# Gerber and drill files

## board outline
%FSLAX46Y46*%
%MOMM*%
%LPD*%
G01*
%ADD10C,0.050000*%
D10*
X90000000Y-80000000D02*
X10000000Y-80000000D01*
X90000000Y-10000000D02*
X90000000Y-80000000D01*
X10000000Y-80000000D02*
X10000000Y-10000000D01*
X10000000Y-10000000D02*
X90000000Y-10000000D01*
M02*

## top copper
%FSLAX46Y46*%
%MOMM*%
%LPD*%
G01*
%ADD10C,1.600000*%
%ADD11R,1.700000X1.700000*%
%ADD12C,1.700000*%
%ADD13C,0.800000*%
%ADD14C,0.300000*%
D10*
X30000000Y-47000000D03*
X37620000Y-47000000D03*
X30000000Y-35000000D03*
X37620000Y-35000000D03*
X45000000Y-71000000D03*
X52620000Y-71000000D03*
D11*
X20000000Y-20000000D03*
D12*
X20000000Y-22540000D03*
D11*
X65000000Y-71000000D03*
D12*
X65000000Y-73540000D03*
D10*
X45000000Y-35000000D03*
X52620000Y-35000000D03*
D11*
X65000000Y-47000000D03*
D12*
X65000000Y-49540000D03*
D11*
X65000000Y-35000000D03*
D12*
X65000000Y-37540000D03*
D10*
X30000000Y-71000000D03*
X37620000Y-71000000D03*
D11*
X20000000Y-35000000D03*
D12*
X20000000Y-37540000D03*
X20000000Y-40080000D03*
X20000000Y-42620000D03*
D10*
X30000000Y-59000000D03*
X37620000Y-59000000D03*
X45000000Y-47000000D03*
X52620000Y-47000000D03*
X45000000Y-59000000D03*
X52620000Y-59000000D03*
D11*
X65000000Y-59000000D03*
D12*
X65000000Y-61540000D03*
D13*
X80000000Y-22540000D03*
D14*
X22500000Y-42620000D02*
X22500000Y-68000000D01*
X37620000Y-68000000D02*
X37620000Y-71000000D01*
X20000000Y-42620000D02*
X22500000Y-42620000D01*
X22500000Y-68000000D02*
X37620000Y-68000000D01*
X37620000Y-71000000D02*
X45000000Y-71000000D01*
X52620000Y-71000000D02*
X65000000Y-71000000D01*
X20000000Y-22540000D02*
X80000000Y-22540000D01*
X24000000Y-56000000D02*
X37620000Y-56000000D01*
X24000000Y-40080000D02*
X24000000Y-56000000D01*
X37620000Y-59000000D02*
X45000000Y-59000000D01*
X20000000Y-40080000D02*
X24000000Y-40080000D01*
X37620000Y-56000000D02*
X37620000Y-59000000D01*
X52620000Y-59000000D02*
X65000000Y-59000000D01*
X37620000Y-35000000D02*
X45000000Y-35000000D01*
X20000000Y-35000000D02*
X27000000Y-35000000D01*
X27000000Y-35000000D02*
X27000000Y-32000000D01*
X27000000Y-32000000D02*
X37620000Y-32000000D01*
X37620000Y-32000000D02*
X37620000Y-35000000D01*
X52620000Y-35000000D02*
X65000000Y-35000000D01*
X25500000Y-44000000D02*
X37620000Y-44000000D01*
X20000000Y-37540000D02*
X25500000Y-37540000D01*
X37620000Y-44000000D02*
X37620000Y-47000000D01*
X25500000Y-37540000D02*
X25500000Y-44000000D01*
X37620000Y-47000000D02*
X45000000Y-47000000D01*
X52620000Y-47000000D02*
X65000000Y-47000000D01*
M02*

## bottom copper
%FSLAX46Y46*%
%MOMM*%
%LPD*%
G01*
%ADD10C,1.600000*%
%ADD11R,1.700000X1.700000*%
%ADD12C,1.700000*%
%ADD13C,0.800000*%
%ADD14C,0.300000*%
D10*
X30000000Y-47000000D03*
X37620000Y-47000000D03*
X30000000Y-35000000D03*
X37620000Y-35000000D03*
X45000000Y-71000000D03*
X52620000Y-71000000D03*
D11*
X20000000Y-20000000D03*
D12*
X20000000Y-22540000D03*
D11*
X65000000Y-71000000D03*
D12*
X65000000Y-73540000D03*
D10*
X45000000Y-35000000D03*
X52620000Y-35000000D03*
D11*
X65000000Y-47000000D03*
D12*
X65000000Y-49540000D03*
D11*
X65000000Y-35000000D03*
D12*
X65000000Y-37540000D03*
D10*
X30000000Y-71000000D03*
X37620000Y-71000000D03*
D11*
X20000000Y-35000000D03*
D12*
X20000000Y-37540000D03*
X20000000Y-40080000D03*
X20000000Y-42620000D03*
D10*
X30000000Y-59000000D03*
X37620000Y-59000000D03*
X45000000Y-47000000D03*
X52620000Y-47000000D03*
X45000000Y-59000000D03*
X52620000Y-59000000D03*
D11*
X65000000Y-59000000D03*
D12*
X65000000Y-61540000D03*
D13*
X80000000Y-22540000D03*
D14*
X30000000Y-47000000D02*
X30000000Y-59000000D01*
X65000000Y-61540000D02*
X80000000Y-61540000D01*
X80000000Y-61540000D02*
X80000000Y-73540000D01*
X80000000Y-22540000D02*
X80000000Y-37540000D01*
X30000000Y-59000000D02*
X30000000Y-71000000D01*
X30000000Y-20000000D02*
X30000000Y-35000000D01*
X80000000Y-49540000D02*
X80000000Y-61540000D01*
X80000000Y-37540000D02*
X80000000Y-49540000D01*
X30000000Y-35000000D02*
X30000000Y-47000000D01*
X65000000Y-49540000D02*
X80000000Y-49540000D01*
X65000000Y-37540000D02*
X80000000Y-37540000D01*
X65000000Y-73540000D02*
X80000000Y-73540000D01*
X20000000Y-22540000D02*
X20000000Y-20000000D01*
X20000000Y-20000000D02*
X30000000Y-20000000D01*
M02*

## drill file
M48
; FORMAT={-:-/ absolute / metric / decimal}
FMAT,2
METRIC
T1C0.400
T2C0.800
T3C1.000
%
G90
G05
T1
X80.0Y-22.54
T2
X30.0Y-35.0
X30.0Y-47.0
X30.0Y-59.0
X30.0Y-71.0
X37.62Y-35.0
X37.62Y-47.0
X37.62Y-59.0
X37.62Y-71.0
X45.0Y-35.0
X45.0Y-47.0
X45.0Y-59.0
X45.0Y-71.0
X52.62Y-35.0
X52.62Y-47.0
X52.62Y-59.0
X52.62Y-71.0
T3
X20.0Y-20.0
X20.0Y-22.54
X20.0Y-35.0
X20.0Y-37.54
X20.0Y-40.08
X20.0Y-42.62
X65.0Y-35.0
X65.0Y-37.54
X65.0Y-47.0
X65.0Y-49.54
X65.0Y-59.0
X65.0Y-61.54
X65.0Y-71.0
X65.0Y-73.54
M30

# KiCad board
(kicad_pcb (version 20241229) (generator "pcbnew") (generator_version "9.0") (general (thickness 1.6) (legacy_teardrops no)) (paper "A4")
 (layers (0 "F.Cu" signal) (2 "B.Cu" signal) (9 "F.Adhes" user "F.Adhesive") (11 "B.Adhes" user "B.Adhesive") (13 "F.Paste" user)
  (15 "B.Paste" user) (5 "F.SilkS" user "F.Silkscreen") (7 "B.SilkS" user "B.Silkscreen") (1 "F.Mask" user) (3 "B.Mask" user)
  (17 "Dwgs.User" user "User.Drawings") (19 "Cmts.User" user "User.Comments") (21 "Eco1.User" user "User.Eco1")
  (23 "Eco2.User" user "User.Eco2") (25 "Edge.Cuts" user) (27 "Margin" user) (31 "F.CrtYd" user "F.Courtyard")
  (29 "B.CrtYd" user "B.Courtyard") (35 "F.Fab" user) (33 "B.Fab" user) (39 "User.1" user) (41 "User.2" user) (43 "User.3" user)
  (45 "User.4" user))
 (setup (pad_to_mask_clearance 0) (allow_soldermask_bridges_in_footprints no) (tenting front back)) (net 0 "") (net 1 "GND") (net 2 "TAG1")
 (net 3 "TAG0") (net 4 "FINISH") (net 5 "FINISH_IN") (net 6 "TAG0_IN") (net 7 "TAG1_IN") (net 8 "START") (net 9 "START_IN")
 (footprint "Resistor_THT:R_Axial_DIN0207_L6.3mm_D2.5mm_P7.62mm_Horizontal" (layer "F.Cu") (at 30 47)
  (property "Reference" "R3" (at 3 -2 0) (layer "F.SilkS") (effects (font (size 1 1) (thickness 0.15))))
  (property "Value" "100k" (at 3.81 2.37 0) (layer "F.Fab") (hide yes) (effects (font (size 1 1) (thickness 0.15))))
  (pad "1" thru_hole circle (at 0 0) (size 1.6 1.6) (drill 0.8) (layers "*.Cu" "*.Mask") (remove_unused_layers no) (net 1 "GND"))
  (pad "2" thru_hole circle (at 7.62 0) (size 1.6 1.6) (drill 0.8) (layers "*.Cu" "*.Mask") (remove_unused_layers no) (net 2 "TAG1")))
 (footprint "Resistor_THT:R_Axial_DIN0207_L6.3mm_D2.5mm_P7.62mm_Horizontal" (layer "F.Cu") (at 30 35)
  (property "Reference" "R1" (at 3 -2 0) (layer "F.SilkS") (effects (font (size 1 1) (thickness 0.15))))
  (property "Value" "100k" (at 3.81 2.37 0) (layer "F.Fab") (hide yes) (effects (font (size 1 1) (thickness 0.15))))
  (pad "1" thru_hole circle (at 0 0) (size 1.6 1.6) (drill 0.8) (layers "*.Cu" "*.Mask") (remove_unused_layers no) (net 1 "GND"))
  (pad "2" thru_hole circle (at 7.62 0) (size 1.6 1.6) (drill 0.8) (layers "*.Cu" "*.Mask") (remove_unused_layers no) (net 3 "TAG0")))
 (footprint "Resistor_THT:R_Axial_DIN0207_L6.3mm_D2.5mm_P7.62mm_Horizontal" (layer "F.Cu") (at 45 71)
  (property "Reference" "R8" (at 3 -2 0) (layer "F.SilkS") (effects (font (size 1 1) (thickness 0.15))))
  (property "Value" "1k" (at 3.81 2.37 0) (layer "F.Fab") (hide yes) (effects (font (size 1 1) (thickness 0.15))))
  (pad "1" thru_hole circle (at 0 0) (size 1.6 1.6) (drill 0.8) (layers "*.Cu" "*.Mask") (remove_unused_layers no) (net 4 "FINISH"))
  (pad "2" thru_hole circle (at 7.62 0) (size 1.6 1.6) (drill 0.8) (layers "*.Cu" "*.Mask") (remove_unused_layers no) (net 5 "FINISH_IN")))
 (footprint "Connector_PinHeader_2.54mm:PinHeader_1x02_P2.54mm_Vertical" (layer "F.Cu") (at 20 20)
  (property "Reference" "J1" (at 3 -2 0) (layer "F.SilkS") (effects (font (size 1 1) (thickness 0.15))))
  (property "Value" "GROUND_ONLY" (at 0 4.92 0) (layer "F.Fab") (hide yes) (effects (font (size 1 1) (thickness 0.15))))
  (pad "1" thru_hole rect (at 0 0) (size 1.7 1.7) (drill 1) (layers "*.Cu" "*.Mask") (remove_unused_layers no) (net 1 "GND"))
  (pad "2" thru_hole circle (at 0 2.54) (size 1.7 1.7) (drill 1) (layers "*.Cu" "*.Mask") (remove_unused_layers no) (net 1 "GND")))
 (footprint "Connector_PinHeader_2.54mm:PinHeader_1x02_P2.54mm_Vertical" (layer "F.Cu") (at 65 71)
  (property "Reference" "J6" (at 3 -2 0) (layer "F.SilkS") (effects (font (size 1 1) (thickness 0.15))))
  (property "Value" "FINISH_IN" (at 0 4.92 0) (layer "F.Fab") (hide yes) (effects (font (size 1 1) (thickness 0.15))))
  (pad "1" thru_hole rect (at 0 0) (size 1.7 1.7) (drill 1) (layers "*.Cu" "*.Mask") (remove_unused_layers no) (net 5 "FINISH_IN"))
  (pad "2" thru_hole circle (at 0 2.54) (size 1.7 1.7) (drill 1) (layers "*.Cu" "*.Mask") (remove_unused_layers no) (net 1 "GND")))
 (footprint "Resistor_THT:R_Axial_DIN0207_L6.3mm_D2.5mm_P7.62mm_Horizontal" (layer "F.Cu") (at 45 35)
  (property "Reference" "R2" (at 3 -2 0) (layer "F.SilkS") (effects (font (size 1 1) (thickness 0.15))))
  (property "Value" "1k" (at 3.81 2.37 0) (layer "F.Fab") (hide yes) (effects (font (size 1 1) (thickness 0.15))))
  (pad "1" thru_hole circle (at 0 0) (size 1.6 1.6) (drill 0.8) (layers "*.Cu" "*.Mask") (remove_unused_layers no) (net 3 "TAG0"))
  (pad "2" thru_hole circle (at 7.62 0) (size 1.6 1.6) (drill 0.8) (layers "*.Cu" "*.Mask") (remove_unused_layers no) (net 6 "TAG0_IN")))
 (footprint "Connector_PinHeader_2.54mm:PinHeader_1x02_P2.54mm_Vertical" (layer "F.Cu") (at 65 47)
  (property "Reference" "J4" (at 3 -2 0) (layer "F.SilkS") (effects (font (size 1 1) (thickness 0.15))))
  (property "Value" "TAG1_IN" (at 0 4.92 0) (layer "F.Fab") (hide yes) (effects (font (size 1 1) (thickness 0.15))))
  (pad "1" thru_hole rect (at 0 0) (size 1.7 1.7) (drill 1) (layers "*.Cu" "*.Mask") (remove_unused_layers no) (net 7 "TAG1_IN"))
  (pad "2" thru_hole circle (at 0 2.54) (size 1.7 1.7) (drill 1) (layers "*.Cu" "*.Mask") (remove_unused_layers no) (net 1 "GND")))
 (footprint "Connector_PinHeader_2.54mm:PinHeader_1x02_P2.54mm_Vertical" (layer "F.Cu") (at 65 35)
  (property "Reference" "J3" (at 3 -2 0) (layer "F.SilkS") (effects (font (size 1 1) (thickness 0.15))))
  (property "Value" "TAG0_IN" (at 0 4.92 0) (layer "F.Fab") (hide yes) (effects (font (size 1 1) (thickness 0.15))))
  (pad "1" thru_hole rect (at 0 0) (size 1.7 1.7) (drill 1) (layers "*.Cu" "*.Mask") (remove_unused_layers no) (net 6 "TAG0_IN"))
  (pad "2" thru_hole circle (at 0 2.54) (size 1.7 1.7) (drill 1) (layers "*.Cu" "*.Mask") (remove_unused_layers no) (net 1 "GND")))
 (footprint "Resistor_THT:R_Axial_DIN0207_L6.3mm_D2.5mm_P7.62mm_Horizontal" (layer "F.Cu") (at 30 71)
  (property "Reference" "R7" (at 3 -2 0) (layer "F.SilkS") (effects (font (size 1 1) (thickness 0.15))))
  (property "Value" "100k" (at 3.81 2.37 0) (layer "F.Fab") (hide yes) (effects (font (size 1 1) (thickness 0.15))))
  (pad "1" thru_hole circle (at 0 0) (size 1.6 1.6) (drill 0.8) (layers "*.Cu" "*.Mask") (remove_unused_layers no) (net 1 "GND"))
  (pad "2" thru_hole circle (at 7.62 0) (size 1.6 1.6) (drill 0.8) (layers "*.Cu" "*.Mask") (remove_unused_layers no) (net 4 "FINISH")))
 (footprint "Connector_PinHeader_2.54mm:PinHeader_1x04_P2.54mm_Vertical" (layer "F.Cu") (at 20 35)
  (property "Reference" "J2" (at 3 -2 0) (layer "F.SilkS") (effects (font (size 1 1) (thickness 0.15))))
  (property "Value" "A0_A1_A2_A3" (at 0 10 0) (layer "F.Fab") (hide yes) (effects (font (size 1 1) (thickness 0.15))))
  (pad "1" thru_hole rect (at 0 0) (size 1.7 1.7) (drill 1) (layers "*.Cu" "*.Mask") (remove_unused_layers no) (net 3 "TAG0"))
  (pad "2" thru_hole circle (at 0 2.54) (size 1.7 1.7) (drill 1) (layers "*.Cu" "*.Mask") (remove_unused_layers no) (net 2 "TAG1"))
  (pad "3" thru_hole circle (at 0 5.08) (size 1.7 1.7) (drill 1) (layers "*.Cu" "*.Mask") (remove_unused_layers no) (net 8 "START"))
  (pad "4" thru_hole circle (at 0 7.62) (size 1.7 1.7) (drill 1) (layers "*.Cu" "*.Mask") (remove_unused_layers no) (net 4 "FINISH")))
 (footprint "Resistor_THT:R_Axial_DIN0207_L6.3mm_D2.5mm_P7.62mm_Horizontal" (layer "F.Cu") (at 30 59)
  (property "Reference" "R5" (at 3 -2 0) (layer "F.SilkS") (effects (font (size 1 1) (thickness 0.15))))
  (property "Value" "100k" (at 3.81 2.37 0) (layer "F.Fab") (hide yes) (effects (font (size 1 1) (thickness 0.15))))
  (pad "1" thru_hole circle (at 0 0) (size 1.6 1.6) (drill 0.8) (layers "*.Cu" "*.Mask") (remove_unused_layers no) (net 1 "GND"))
  (pad "2" thru_hole circle (at 7.62 0) (size 1.6 1.6) (drill 0.8) (layers "*.Cu" "*.Mask") (remove_unused_layers no) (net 8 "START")))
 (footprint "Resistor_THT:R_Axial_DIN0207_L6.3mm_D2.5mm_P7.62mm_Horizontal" (layer "F.Cu") (at 45 47)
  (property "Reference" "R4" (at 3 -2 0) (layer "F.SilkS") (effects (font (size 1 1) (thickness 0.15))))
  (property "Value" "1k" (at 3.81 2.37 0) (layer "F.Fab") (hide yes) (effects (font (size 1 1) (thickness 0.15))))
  (pad "1" thru_hole circle (at 0 0) (size 1.6 1.6) (drill 0.8) (layers "*.Cu" "*.Mask") (remove_unused_layers no) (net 2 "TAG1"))
  (pad "2" thru_hole circle (at 7.62 0) (size 1.6 1.6) (drill 0.8) (layers "*.Cu" "*.Mask") (remove_unused_layers no) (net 7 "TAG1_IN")))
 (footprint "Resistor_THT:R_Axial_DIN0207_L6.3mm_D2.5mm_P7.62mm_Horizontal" (layer "F.Cu") (at 45 59)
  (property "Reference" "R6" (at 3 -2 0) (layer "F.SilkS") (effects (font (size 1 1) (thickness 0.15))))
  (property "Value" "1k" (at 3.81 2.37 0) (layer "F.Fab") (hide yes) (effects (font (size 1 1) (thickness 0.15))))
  (pad "1" thru_hole circle (at 0 0) (size 1.6 1.6) (drill 0.8) (layers "*.Cu" "*.Mask") (remove_unused_layers no) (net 8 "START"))
  (pad "2" thru_hole circle (at 7.62 0) (size 1.6 1.6) (drill 0.8) (layers "*.Cu" "*.Mask") (remove_unused_layers no) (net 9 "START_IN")))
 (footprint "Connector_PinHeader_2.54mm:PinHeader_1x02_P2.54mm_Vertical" (layer "F.Cu") (at 65 59)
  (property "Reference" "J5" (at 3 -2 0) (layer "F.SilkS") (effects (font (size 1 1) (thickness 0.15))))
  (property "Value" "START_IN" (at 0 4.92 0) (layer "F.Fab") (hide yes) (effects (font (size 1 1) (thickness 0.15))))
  (pad "1" thru_hole rect (at 0 0) (size 1.7 1.7) (drill 1) (layers "*.Cu" "*.Mask") (remove_unused_layers no) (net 9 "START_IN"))
  (pad "2" thru_hole circle (at 0 2.54) (size 1.7 1.7) (drill 1) (layers "*.Cu" "*.Mask") (remove_unused_layers no) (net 1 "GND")))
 (gr_line (start 90 80) (end 10 80) (stroke (width 0.05) (type default)) (layer "Edge.Cuts"))
 (gr_line (start 90 10) (end 90 80) (stroke (width 0.05) (type default)) (layer "Edge.Cuts"))
 (gr_line (start 10 80) (end 10 10) (stroke (width 0.05) (type default)) (layer "Edge.Cuts"))
 (gr_line (start 10 10) (end 90 10) (stroke (width 0.05) (type default)) (layer "Edge.Cuts"))
 (segment (start 22.5 42.62) (end 22.5 68) (width 0.3) (layer "F.Cu") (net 4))
 (segment (start 37.62 68) (end 37.62 71) (width 0.3) (layer "F.Cu") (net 4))
 (segment (start 20 42.62) (end 22.5 42.62) (width 0.3) (layer "F.Cu") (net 4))
 (segment (start 22.5 68) (end 37.62 68) (width 0.3) (layer "F.Cu") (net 4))
 (segment (start 37.62 71) (end 45 71) (width 0.3) (layer "F.Cu") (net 4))
 (segment (start 52.62 71) (end 65 71) (width 0.3) (layer "F.Cu") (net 5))
 (segment (start 20 22.54) (end 80 22.54) (width 0.3) (layer "F.Cu") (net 1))
 (via (at 80 22.54) (size 0.8) (drill 0.4) (layers "F.Cu" "B.Cu") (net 1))
 (segment (start 30 47) (end 30 59) (width 0.3) (layer "B.Cu") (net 1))
 (segment (start 65 61.54) (end 80 61.54) (width 0.3) (layer "B.Cu") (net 1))
 (segment (start 80 61.54) (end 80 73.54) (width 0.3) (layer "B.Cu") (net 1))
 (segment (start 80 22.54) (end 80 37.54) (width 0.3) (layer "B.Cu") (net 1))
 (segment (start 30 59) (end 30 71) (width 0.3) (layer "B.Cu") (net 1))
 (segment (start 30 20) (end 30 35) (width 0.3) (layer "B.Cu") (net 1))
 (segment (start 80 49.54) (end 80 61.54) (width 0.3) (layer "B.Cu") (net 1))
 (segment (start 80 37.54) (end 80 49.54) (width 0.3) (layer "B.Cu") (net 1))
 (segment (start 30 35) (end 30 47) (width 0.3) (layer "B.Cu") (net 1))
 (segment (start 65 49.54) (end 80 49.54) (width 0.3) (layer "B.Cu") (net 1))
 (segment (start 65 37.54) (end 80 37.54) (width 0.3) (layer "B.Cu") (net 1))
 (segment (start 65 73.54) (end 80 73.54) (width 0.3) (layer "B.Cu") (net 1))
 (segment (start 20 22.54) (end 20 20) (width 0.3) (layer "B.Cu") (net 1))
 (segment (start 20 20) (end 30 20) (width 0.3) (layer "B.Cu") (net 1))
 (segment (start 24 56) (end 37.62 56) (width 0.3) (layer "F.Cu") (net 8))
 (segment (start 24 40.08) (end 24 56) (width 0.3) (layer "F.Cu") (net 8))
 (segment (start 37.62 59) (end 45 59) (width 0.3) (layer "F.Cu") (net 8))
 (segment (start 20 40.08) (end 24 40.08) (width 0.3) (layer "F.Cu") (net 8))
 (segment (start 37.62 56) (end 37.62 59) (width 0.3) (layer "F.Cu") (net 8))
 (segment (start 52.62 59) (end 65 59) (width 0.3) (layer "F.Cu") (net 9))
 (segment (start 37.62 35) (end 45 35) (width 0.3) (layer "F.Cu") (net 3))
 (segment (start 20 35) (end 27 35) (width 0.3) (layer "F.Cu") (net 3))
 (segment (start 27 35) (end 27 32) (width 0.3) (layer "F.Cu") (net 3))
 (segment (start 27 32) (end 37.62 32) (width 0.3) (layer "F.Cu") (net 3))
 (segment (start 37.62 32) (end 37.62 35) (width 0.3) (layer "F.Cu") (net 3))
 (segment (start 52.62 35) (end 65 35) (width 0.3) (layer "F.Cu") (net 6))
 (segment (start 25.5 44) (end 37.62 44) (width 0.3) (layer "F.Cu") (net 2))
 (segment (start 20 37.54) (end 25.5 37.54) (width 0.3) (layer "F.Cu") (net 2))
 (segment (start 37.62 44) (end 37.62 47) (width 0.3) (layer "F.Cu") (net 2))
 (segment (start 25.5 37.54) (end 25.5 44) (width 0.3) (layer "F.Cu") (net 2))
 (segment (start 37.62 47) (end 45 47) (width 0.3) (layer "F.Cu") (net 2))
 (segment (start 52.62 47) (end 65 47) (width 0.3) (layer "F.Cu") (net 7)))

